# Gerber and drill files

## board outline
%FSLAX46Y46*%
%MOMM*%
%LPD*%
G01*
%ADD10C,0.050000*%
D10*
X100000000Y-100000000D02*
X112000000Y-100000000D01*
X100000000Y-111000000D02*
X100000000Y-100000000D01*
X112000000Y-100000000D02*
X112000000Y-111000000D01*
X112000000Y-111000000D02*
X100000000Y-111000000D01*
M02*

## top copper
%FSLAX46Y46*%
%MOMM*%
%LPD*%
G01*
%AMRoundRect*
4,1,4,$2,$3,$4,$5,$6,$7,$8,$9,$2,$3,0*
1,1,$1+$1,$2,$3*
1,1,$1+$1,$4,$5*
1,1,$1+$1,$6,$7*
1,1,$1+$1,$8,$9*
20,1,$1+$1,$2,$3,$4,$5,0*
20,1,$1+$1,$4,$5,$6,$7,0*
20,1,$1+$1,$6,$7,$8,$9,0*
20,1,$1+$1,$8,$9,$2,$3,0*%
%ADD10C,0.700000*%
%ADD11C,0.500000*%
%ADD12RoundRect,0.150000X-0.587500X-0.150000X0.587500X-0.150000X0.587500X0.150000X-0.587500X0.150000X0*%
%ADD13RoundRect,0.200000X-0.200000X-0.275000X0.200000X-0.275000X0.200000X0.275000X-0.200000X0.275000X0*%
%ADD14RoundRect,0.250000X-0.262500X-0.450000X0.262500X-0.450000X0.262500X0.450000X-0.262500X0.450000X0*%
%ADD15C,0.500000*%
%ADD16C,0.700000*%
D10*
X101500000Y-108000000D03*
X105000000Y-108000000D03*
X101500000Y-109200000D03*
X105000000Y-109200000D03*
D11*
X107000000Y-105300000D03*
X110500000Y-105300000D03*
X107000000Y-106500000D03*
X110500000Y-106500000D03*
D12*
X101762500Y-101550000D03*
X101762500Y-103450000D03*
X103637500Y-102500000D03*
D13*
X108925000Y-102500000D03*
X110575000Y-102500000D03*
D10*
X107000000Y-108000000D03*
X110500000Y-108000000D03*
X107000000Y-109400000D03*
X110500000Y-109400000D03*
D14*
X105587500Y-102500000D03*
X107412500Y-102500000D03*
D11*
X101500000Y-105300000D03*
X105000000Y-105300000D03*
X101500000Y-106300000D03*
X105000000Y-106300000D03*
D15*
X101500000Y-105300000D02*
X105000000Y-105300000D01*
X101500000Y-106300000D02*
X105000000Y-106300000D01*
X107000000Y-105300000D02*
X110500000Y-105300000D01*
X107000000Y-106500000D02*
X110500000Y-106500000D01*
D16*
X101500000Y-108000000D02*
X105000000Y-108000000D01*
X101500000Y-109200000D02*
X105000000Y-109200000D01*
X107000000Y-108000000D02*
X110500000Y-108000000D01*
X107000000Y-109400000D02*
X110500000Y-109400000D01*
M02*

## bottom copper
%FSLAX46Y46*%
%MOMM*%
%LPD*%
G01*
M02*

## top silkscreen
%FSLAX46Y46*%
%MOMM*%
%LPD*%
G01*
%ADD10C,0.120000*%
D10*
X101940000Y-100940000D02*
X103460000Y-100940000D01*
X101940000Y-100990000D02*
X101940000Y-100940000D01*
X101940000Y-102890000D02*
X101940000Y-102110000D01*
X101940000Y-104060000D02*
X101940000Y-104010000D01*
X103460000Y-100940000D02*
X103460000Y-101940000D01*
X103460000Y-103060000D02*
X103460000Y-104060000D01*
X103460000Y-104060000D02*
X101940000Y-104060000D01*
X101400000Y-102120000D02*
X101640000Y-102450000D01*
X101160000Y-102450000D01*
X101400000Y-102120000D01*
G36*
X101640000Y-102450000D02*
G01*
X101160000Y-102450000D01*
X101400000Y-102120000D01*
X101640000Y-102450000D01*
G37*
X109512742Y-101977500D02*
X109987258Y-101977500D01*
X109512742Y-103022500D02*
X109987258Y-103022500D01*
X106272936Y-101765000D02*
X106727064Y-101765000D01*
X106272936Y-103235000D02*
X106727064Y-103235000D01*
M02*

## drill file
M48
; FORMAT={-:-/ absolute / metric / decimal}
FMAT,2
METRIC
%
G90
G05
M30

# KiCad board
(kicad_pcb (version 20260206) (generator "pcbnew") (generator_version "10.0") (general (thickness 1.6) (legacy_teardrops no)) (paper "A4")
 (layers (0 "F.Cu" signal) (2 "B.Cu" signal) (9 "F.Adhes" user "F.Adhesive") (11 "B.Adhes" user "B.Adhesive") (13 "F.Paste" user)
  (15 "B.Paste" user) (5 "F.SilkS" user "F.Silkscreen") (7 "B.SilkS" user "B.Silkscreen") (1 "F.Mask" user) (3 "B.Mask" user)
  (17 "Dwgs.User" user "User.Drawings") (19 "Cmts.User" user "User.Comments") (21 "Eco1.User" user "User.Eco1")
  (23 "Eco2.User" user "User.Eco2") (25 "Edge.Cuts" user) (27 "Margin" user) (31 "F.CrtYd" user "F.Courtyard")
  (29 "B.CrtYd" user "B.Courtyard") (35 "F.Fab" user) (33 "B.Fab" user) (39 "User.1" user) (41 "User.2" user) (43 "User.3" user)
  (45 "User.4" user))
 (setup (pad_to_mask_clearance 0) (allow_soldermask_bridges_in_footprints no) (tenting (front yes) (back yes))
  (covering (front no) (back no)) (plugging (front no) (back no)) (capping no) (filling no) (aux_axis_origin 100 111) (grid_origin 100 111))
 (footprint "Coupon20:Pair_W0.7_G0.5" (layer "F.Cu") (at 101.5 108)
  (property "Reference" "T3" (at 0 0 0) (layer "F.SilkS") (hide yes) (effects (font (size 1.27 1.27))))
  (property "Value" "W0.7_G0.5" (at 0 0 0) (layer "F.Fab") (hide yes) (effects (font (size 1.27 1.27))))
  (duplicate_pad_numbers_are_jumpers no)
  (pad "1" smd circle (at 0 0) (size 0.7 0.7) (layers "F.Cu" "F.Mask") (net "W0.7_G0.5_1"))
  (pad "2" smd circle (at 3.5 0) (size 0.7 0.7) (layers "F.Cu" "F.Mask") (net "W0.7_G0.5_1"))
  (pad "3" smd circle (at 0 1.2) (size 0.7 0.7) (layers "F.Cu" "F.Mask") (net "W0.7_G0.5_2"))
  (pad "4" smd circle (at 3.5 1.2) (size 0.7 0.7) (layers "F.Cu" "F.Mask") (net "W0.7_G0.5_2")))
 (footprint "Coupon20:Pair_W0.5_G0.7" (layer "F.Cu") (at 107 105.3)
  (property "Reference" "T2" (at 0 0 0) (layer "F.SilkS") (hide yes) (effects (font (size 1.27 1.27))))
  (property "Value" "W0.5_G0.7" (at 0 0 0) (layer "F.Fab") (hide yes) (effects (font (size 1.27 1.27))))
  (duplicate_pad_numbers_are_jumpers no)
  (pad "1" smd circle (at 0 0) (size 0.5 0.5) (layers "F.Cu" "F.Mask") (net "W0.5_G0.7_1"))
  (pad "2" smd circle (at 3.5 0) (size 0.5 0.5) (layers "F.Cu" "F.Mask") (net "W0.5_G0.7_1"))
  (pad "3" smd circle (at 0 1.2) (size 0.5 0.5) (layers "F.Cu" "F.Mask") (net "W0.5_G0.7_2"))
  (pad "4" smd circle (at 3.5 1.2) (size 0.5 0.5) (layers "F.Cu" "F.Mask") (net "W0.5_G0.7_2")))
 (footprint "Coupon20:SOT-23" (layer "F.Cu") (at 102.7 102.5)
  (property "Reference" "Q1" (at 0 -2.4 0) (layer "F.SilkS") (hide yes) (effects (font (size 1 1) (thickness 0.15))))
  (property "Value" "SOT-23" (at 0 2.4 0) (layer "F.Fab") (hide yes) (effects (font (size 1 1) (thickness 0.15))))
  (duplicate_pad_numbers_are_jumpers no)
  (fp_line (start -0.76 -1.56) (end 0.76 -1.56) (stroke (width 0.12) (type solid)) (layer "F.SilkS"))
  (fp_line (start -0.76 -1.51) (end -0.76 -1.56) (stroke (width 0.12) (type solid)) (layer "F.SilkS"))
  (fp_line (start -0.76 0.39) (end -0.76 -0.39) (stroke (width 0.12) (type solid)) (layer "F.SilkS"))
  (fp_line (start -0.76 1.56) (end -0.76 1.51) (stroke (width 0.12) (type solid)) (layer "F.SilkS"))
  (fp_line (start 0.76 -1.56) (end 0.76 -0.56) (stroke (width 0.12) (type solid)) (layer "F.SilkS"))
  (fp_line (start 0.76 0.56) (end 0.76 1.56) (stroke (width 0.12) (type solid)) (layer "F.SilkS"))
  (fp_line (start 0.76 1.56) (end -0.76 1.56) (stroke (width 0.12) (type solid)) (layer "F.SilkS"))
  (fp_poly (pts (xy -1.3 -0.38) (xy -1.06 -0.05) (xy -1.54 -0.05)) (stroke (width 0.12) (type solid)) (fill yes) (layer "F.SilkS"))
  (pad "1" smd roundrect (at -0.9375 -0.95) (size 1.475 0.6) (layers "F.Cu" "F.Mask" "F.Paste") (roundrect_rratio 0.25) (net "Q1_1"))
  (pad "2" smd roundrect (at -0.9375 0.95) (size 1.475 0.6) (layers "F.Cu" "F.Mask" "F.Paste") (roundrect_rratio 0.25) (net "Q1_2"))
  (pad "3" smd roundrect (at 0.9375 0) (size 1.475 0.6) (layers "F.Cu" "F.Mask" "F.Paste") (roundrect_rratio 0.25) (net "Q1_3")))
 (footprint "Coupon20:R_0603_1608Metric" (layer "F.Cu") (at 109.75 102.5)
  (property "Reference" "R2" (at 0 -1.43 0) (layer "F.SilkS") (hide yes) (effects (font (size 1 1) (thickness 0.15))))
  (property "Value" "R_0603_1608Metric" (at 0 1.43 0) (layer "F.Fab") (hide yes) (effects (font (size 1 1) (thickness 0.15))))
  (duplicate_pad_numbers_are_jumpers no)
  (fp_line (start -0.237258 -0.5225) (end 0.237258 -0.5225) (stroke (width 0.12) (type solid)) (layer "F.SilkS"))
  (fp_line (start -0.237258 0.5225) (end 0.237258 0.5225) (stroke (width 0.12) (type solid)) (layer "F.SilkS"))
  (pad "1" smd roundrect (at -0.825 0) (size 0.8 0.95) (layers "F.Cu" "F.Mask" "F.Paste") (roundrect_rratio 0.25) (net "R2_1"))
  (pad "2" smd roundrect (at 0.825 0) (size 0.8 0.95) (layers "F.Cu" "F.Mask" "F.Paste") (roundrect_rratio 0.25) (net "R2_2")))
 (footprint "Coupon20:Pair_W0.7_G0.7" (layer "F.Cu") (at 107 108)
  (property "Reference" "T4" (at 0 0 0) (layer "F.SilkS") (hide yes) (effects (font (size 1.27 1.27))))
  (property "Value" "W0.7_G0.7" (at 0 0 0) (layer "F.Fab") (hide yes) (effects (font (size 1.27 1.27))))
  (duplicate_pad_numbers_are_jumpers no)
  (pad "1" smd circle (at 0 0) (size 0.7 0.7) (layers "F.Cu" "F.Mask") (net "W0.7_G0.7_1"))
  (pad "2" smd circle (at 3.5 0) (size 0.7 0.7) (layers "F.Cu" "F.Mask") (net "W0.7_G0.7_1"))
  (pad "3" smd circle (at 0 1.4) (size 0.7 0.7) (layers "F.Cu" "F.Mask") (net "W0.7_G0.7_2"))
  (pad "4" smd circle (at 3.5 1.4) (size 0.7 0.7) (layers "F.Cu" "F.Mask") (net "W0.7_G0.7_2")))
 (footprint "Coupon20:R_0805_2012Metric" (layer "F.Cu") (at 106.5 102.5)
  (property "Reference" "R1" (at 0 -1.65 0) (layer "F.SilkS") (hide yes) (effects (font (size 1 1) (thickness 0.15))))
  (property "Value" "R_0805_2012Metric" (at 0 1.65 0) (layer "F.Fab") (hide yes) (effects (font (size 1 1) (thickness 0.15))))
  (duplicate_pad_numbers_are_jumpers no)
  (fp_line (start -0.227064 -0.735) (end 0.227064 -0.735) (stroke (width 0.12) (type solid)) (layer "F.SilkS"))
  (fp_line (start -0.227064 0.735) (end 0.227064 0.735) (stroke (width 0.12) (type solid)) (layer "F.SilkS"))
  (pad "1" smd roundrect (at -0.9125 0) (size 1.025 1.4) (layers "F.Cu" "F.Mask" "F.Paste") (roundrect_rratio 0.243902) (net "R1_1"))
  (pad "2" smd roundrect (at 0.9125 0) (size 1.025 1.4) (layers "F.Cu" "F.Mask" "F.Paste") (roundrect_rratio 0.243902) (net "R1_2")))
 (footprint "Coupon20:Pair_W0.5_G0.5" (layer "F.Cu") (at 101.5 105.3)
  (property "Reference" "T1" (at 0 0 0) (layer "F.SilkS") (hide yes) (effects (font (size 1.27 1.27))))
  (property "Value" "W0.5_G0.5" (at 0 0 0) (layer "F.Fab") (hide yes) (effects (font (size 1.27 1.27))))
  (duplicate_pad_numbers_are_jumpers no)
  (pad "1" smd circle (at 0 0) (size 0.5 0.5) (layers "F.Cu" "F.Mask") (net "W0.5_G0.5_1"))
  (pad "2" smd circle (at 3.5 0) (size 0.5 0.5) (layers "F.Cu" "F.Mask") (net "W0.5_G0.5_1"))
  (pad "3" smd circle (at 0 1) (size 0.5 0.5) (layers "F.Cu" "F.Mask") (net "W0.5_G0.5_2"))
  (pad "4" smd circle (at 3.5 1) (size 0.5 0.5) (layers "F.Cu" "F.Mask") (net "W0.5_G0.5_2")))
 (gr_line (start 100 100) (end 112 100) (stroke (width 0.05) (type default)) (layer "Edge.Cuts"))
 (gr_line (start 100 111) (end 100 100) (stroke (width 0.05) (type default)) (layer "Edge.Cuts"))
 (gr_line (start 112 100) (end 112 111) (stroke (width 0.05) (type default)) (layer "Edge.Cuts"))
 (gr_line (start 112 111) (end 100 111) (stroke (width 0.05) (type default)) (layer "Edge.Cuts"))
 (segment (start 101.5 105.3) (end 105 105.3) (width 0.5) (layer "F.Cu") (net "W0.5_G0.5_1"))
 (segment (start 101.5 106.3) (end 105 106.3) (width 0.5) (layer "F.Cu") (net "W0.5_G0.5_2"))
 (segment (start 107 105.3) (end 110.5 105.3) (width 0.5) (layer "F.Cu") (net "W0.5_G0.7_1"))
 (segment (start 107 106.5) (end 110.5 106.5) (width 0.5) (layer "F.Cu") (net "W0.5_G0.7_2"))
 (segment (start 101.5 108) (end 105 108) (width 0.7) (layer "F.Cu") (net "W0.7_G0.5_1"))
 (segment (start 101.5 109.2) (end 105 109.2) (width 0.7) (layer "F.Cu") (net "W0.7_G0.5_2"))
 (segment (start 107 108) (end 110.5 108) (width 0.7) (layer "F.Cu") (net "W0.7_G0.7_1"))
 (segment (start 107 109.4) (end 110.5 109.4) (width 0.7) (layer "F.Cu") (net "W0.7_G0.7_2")))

